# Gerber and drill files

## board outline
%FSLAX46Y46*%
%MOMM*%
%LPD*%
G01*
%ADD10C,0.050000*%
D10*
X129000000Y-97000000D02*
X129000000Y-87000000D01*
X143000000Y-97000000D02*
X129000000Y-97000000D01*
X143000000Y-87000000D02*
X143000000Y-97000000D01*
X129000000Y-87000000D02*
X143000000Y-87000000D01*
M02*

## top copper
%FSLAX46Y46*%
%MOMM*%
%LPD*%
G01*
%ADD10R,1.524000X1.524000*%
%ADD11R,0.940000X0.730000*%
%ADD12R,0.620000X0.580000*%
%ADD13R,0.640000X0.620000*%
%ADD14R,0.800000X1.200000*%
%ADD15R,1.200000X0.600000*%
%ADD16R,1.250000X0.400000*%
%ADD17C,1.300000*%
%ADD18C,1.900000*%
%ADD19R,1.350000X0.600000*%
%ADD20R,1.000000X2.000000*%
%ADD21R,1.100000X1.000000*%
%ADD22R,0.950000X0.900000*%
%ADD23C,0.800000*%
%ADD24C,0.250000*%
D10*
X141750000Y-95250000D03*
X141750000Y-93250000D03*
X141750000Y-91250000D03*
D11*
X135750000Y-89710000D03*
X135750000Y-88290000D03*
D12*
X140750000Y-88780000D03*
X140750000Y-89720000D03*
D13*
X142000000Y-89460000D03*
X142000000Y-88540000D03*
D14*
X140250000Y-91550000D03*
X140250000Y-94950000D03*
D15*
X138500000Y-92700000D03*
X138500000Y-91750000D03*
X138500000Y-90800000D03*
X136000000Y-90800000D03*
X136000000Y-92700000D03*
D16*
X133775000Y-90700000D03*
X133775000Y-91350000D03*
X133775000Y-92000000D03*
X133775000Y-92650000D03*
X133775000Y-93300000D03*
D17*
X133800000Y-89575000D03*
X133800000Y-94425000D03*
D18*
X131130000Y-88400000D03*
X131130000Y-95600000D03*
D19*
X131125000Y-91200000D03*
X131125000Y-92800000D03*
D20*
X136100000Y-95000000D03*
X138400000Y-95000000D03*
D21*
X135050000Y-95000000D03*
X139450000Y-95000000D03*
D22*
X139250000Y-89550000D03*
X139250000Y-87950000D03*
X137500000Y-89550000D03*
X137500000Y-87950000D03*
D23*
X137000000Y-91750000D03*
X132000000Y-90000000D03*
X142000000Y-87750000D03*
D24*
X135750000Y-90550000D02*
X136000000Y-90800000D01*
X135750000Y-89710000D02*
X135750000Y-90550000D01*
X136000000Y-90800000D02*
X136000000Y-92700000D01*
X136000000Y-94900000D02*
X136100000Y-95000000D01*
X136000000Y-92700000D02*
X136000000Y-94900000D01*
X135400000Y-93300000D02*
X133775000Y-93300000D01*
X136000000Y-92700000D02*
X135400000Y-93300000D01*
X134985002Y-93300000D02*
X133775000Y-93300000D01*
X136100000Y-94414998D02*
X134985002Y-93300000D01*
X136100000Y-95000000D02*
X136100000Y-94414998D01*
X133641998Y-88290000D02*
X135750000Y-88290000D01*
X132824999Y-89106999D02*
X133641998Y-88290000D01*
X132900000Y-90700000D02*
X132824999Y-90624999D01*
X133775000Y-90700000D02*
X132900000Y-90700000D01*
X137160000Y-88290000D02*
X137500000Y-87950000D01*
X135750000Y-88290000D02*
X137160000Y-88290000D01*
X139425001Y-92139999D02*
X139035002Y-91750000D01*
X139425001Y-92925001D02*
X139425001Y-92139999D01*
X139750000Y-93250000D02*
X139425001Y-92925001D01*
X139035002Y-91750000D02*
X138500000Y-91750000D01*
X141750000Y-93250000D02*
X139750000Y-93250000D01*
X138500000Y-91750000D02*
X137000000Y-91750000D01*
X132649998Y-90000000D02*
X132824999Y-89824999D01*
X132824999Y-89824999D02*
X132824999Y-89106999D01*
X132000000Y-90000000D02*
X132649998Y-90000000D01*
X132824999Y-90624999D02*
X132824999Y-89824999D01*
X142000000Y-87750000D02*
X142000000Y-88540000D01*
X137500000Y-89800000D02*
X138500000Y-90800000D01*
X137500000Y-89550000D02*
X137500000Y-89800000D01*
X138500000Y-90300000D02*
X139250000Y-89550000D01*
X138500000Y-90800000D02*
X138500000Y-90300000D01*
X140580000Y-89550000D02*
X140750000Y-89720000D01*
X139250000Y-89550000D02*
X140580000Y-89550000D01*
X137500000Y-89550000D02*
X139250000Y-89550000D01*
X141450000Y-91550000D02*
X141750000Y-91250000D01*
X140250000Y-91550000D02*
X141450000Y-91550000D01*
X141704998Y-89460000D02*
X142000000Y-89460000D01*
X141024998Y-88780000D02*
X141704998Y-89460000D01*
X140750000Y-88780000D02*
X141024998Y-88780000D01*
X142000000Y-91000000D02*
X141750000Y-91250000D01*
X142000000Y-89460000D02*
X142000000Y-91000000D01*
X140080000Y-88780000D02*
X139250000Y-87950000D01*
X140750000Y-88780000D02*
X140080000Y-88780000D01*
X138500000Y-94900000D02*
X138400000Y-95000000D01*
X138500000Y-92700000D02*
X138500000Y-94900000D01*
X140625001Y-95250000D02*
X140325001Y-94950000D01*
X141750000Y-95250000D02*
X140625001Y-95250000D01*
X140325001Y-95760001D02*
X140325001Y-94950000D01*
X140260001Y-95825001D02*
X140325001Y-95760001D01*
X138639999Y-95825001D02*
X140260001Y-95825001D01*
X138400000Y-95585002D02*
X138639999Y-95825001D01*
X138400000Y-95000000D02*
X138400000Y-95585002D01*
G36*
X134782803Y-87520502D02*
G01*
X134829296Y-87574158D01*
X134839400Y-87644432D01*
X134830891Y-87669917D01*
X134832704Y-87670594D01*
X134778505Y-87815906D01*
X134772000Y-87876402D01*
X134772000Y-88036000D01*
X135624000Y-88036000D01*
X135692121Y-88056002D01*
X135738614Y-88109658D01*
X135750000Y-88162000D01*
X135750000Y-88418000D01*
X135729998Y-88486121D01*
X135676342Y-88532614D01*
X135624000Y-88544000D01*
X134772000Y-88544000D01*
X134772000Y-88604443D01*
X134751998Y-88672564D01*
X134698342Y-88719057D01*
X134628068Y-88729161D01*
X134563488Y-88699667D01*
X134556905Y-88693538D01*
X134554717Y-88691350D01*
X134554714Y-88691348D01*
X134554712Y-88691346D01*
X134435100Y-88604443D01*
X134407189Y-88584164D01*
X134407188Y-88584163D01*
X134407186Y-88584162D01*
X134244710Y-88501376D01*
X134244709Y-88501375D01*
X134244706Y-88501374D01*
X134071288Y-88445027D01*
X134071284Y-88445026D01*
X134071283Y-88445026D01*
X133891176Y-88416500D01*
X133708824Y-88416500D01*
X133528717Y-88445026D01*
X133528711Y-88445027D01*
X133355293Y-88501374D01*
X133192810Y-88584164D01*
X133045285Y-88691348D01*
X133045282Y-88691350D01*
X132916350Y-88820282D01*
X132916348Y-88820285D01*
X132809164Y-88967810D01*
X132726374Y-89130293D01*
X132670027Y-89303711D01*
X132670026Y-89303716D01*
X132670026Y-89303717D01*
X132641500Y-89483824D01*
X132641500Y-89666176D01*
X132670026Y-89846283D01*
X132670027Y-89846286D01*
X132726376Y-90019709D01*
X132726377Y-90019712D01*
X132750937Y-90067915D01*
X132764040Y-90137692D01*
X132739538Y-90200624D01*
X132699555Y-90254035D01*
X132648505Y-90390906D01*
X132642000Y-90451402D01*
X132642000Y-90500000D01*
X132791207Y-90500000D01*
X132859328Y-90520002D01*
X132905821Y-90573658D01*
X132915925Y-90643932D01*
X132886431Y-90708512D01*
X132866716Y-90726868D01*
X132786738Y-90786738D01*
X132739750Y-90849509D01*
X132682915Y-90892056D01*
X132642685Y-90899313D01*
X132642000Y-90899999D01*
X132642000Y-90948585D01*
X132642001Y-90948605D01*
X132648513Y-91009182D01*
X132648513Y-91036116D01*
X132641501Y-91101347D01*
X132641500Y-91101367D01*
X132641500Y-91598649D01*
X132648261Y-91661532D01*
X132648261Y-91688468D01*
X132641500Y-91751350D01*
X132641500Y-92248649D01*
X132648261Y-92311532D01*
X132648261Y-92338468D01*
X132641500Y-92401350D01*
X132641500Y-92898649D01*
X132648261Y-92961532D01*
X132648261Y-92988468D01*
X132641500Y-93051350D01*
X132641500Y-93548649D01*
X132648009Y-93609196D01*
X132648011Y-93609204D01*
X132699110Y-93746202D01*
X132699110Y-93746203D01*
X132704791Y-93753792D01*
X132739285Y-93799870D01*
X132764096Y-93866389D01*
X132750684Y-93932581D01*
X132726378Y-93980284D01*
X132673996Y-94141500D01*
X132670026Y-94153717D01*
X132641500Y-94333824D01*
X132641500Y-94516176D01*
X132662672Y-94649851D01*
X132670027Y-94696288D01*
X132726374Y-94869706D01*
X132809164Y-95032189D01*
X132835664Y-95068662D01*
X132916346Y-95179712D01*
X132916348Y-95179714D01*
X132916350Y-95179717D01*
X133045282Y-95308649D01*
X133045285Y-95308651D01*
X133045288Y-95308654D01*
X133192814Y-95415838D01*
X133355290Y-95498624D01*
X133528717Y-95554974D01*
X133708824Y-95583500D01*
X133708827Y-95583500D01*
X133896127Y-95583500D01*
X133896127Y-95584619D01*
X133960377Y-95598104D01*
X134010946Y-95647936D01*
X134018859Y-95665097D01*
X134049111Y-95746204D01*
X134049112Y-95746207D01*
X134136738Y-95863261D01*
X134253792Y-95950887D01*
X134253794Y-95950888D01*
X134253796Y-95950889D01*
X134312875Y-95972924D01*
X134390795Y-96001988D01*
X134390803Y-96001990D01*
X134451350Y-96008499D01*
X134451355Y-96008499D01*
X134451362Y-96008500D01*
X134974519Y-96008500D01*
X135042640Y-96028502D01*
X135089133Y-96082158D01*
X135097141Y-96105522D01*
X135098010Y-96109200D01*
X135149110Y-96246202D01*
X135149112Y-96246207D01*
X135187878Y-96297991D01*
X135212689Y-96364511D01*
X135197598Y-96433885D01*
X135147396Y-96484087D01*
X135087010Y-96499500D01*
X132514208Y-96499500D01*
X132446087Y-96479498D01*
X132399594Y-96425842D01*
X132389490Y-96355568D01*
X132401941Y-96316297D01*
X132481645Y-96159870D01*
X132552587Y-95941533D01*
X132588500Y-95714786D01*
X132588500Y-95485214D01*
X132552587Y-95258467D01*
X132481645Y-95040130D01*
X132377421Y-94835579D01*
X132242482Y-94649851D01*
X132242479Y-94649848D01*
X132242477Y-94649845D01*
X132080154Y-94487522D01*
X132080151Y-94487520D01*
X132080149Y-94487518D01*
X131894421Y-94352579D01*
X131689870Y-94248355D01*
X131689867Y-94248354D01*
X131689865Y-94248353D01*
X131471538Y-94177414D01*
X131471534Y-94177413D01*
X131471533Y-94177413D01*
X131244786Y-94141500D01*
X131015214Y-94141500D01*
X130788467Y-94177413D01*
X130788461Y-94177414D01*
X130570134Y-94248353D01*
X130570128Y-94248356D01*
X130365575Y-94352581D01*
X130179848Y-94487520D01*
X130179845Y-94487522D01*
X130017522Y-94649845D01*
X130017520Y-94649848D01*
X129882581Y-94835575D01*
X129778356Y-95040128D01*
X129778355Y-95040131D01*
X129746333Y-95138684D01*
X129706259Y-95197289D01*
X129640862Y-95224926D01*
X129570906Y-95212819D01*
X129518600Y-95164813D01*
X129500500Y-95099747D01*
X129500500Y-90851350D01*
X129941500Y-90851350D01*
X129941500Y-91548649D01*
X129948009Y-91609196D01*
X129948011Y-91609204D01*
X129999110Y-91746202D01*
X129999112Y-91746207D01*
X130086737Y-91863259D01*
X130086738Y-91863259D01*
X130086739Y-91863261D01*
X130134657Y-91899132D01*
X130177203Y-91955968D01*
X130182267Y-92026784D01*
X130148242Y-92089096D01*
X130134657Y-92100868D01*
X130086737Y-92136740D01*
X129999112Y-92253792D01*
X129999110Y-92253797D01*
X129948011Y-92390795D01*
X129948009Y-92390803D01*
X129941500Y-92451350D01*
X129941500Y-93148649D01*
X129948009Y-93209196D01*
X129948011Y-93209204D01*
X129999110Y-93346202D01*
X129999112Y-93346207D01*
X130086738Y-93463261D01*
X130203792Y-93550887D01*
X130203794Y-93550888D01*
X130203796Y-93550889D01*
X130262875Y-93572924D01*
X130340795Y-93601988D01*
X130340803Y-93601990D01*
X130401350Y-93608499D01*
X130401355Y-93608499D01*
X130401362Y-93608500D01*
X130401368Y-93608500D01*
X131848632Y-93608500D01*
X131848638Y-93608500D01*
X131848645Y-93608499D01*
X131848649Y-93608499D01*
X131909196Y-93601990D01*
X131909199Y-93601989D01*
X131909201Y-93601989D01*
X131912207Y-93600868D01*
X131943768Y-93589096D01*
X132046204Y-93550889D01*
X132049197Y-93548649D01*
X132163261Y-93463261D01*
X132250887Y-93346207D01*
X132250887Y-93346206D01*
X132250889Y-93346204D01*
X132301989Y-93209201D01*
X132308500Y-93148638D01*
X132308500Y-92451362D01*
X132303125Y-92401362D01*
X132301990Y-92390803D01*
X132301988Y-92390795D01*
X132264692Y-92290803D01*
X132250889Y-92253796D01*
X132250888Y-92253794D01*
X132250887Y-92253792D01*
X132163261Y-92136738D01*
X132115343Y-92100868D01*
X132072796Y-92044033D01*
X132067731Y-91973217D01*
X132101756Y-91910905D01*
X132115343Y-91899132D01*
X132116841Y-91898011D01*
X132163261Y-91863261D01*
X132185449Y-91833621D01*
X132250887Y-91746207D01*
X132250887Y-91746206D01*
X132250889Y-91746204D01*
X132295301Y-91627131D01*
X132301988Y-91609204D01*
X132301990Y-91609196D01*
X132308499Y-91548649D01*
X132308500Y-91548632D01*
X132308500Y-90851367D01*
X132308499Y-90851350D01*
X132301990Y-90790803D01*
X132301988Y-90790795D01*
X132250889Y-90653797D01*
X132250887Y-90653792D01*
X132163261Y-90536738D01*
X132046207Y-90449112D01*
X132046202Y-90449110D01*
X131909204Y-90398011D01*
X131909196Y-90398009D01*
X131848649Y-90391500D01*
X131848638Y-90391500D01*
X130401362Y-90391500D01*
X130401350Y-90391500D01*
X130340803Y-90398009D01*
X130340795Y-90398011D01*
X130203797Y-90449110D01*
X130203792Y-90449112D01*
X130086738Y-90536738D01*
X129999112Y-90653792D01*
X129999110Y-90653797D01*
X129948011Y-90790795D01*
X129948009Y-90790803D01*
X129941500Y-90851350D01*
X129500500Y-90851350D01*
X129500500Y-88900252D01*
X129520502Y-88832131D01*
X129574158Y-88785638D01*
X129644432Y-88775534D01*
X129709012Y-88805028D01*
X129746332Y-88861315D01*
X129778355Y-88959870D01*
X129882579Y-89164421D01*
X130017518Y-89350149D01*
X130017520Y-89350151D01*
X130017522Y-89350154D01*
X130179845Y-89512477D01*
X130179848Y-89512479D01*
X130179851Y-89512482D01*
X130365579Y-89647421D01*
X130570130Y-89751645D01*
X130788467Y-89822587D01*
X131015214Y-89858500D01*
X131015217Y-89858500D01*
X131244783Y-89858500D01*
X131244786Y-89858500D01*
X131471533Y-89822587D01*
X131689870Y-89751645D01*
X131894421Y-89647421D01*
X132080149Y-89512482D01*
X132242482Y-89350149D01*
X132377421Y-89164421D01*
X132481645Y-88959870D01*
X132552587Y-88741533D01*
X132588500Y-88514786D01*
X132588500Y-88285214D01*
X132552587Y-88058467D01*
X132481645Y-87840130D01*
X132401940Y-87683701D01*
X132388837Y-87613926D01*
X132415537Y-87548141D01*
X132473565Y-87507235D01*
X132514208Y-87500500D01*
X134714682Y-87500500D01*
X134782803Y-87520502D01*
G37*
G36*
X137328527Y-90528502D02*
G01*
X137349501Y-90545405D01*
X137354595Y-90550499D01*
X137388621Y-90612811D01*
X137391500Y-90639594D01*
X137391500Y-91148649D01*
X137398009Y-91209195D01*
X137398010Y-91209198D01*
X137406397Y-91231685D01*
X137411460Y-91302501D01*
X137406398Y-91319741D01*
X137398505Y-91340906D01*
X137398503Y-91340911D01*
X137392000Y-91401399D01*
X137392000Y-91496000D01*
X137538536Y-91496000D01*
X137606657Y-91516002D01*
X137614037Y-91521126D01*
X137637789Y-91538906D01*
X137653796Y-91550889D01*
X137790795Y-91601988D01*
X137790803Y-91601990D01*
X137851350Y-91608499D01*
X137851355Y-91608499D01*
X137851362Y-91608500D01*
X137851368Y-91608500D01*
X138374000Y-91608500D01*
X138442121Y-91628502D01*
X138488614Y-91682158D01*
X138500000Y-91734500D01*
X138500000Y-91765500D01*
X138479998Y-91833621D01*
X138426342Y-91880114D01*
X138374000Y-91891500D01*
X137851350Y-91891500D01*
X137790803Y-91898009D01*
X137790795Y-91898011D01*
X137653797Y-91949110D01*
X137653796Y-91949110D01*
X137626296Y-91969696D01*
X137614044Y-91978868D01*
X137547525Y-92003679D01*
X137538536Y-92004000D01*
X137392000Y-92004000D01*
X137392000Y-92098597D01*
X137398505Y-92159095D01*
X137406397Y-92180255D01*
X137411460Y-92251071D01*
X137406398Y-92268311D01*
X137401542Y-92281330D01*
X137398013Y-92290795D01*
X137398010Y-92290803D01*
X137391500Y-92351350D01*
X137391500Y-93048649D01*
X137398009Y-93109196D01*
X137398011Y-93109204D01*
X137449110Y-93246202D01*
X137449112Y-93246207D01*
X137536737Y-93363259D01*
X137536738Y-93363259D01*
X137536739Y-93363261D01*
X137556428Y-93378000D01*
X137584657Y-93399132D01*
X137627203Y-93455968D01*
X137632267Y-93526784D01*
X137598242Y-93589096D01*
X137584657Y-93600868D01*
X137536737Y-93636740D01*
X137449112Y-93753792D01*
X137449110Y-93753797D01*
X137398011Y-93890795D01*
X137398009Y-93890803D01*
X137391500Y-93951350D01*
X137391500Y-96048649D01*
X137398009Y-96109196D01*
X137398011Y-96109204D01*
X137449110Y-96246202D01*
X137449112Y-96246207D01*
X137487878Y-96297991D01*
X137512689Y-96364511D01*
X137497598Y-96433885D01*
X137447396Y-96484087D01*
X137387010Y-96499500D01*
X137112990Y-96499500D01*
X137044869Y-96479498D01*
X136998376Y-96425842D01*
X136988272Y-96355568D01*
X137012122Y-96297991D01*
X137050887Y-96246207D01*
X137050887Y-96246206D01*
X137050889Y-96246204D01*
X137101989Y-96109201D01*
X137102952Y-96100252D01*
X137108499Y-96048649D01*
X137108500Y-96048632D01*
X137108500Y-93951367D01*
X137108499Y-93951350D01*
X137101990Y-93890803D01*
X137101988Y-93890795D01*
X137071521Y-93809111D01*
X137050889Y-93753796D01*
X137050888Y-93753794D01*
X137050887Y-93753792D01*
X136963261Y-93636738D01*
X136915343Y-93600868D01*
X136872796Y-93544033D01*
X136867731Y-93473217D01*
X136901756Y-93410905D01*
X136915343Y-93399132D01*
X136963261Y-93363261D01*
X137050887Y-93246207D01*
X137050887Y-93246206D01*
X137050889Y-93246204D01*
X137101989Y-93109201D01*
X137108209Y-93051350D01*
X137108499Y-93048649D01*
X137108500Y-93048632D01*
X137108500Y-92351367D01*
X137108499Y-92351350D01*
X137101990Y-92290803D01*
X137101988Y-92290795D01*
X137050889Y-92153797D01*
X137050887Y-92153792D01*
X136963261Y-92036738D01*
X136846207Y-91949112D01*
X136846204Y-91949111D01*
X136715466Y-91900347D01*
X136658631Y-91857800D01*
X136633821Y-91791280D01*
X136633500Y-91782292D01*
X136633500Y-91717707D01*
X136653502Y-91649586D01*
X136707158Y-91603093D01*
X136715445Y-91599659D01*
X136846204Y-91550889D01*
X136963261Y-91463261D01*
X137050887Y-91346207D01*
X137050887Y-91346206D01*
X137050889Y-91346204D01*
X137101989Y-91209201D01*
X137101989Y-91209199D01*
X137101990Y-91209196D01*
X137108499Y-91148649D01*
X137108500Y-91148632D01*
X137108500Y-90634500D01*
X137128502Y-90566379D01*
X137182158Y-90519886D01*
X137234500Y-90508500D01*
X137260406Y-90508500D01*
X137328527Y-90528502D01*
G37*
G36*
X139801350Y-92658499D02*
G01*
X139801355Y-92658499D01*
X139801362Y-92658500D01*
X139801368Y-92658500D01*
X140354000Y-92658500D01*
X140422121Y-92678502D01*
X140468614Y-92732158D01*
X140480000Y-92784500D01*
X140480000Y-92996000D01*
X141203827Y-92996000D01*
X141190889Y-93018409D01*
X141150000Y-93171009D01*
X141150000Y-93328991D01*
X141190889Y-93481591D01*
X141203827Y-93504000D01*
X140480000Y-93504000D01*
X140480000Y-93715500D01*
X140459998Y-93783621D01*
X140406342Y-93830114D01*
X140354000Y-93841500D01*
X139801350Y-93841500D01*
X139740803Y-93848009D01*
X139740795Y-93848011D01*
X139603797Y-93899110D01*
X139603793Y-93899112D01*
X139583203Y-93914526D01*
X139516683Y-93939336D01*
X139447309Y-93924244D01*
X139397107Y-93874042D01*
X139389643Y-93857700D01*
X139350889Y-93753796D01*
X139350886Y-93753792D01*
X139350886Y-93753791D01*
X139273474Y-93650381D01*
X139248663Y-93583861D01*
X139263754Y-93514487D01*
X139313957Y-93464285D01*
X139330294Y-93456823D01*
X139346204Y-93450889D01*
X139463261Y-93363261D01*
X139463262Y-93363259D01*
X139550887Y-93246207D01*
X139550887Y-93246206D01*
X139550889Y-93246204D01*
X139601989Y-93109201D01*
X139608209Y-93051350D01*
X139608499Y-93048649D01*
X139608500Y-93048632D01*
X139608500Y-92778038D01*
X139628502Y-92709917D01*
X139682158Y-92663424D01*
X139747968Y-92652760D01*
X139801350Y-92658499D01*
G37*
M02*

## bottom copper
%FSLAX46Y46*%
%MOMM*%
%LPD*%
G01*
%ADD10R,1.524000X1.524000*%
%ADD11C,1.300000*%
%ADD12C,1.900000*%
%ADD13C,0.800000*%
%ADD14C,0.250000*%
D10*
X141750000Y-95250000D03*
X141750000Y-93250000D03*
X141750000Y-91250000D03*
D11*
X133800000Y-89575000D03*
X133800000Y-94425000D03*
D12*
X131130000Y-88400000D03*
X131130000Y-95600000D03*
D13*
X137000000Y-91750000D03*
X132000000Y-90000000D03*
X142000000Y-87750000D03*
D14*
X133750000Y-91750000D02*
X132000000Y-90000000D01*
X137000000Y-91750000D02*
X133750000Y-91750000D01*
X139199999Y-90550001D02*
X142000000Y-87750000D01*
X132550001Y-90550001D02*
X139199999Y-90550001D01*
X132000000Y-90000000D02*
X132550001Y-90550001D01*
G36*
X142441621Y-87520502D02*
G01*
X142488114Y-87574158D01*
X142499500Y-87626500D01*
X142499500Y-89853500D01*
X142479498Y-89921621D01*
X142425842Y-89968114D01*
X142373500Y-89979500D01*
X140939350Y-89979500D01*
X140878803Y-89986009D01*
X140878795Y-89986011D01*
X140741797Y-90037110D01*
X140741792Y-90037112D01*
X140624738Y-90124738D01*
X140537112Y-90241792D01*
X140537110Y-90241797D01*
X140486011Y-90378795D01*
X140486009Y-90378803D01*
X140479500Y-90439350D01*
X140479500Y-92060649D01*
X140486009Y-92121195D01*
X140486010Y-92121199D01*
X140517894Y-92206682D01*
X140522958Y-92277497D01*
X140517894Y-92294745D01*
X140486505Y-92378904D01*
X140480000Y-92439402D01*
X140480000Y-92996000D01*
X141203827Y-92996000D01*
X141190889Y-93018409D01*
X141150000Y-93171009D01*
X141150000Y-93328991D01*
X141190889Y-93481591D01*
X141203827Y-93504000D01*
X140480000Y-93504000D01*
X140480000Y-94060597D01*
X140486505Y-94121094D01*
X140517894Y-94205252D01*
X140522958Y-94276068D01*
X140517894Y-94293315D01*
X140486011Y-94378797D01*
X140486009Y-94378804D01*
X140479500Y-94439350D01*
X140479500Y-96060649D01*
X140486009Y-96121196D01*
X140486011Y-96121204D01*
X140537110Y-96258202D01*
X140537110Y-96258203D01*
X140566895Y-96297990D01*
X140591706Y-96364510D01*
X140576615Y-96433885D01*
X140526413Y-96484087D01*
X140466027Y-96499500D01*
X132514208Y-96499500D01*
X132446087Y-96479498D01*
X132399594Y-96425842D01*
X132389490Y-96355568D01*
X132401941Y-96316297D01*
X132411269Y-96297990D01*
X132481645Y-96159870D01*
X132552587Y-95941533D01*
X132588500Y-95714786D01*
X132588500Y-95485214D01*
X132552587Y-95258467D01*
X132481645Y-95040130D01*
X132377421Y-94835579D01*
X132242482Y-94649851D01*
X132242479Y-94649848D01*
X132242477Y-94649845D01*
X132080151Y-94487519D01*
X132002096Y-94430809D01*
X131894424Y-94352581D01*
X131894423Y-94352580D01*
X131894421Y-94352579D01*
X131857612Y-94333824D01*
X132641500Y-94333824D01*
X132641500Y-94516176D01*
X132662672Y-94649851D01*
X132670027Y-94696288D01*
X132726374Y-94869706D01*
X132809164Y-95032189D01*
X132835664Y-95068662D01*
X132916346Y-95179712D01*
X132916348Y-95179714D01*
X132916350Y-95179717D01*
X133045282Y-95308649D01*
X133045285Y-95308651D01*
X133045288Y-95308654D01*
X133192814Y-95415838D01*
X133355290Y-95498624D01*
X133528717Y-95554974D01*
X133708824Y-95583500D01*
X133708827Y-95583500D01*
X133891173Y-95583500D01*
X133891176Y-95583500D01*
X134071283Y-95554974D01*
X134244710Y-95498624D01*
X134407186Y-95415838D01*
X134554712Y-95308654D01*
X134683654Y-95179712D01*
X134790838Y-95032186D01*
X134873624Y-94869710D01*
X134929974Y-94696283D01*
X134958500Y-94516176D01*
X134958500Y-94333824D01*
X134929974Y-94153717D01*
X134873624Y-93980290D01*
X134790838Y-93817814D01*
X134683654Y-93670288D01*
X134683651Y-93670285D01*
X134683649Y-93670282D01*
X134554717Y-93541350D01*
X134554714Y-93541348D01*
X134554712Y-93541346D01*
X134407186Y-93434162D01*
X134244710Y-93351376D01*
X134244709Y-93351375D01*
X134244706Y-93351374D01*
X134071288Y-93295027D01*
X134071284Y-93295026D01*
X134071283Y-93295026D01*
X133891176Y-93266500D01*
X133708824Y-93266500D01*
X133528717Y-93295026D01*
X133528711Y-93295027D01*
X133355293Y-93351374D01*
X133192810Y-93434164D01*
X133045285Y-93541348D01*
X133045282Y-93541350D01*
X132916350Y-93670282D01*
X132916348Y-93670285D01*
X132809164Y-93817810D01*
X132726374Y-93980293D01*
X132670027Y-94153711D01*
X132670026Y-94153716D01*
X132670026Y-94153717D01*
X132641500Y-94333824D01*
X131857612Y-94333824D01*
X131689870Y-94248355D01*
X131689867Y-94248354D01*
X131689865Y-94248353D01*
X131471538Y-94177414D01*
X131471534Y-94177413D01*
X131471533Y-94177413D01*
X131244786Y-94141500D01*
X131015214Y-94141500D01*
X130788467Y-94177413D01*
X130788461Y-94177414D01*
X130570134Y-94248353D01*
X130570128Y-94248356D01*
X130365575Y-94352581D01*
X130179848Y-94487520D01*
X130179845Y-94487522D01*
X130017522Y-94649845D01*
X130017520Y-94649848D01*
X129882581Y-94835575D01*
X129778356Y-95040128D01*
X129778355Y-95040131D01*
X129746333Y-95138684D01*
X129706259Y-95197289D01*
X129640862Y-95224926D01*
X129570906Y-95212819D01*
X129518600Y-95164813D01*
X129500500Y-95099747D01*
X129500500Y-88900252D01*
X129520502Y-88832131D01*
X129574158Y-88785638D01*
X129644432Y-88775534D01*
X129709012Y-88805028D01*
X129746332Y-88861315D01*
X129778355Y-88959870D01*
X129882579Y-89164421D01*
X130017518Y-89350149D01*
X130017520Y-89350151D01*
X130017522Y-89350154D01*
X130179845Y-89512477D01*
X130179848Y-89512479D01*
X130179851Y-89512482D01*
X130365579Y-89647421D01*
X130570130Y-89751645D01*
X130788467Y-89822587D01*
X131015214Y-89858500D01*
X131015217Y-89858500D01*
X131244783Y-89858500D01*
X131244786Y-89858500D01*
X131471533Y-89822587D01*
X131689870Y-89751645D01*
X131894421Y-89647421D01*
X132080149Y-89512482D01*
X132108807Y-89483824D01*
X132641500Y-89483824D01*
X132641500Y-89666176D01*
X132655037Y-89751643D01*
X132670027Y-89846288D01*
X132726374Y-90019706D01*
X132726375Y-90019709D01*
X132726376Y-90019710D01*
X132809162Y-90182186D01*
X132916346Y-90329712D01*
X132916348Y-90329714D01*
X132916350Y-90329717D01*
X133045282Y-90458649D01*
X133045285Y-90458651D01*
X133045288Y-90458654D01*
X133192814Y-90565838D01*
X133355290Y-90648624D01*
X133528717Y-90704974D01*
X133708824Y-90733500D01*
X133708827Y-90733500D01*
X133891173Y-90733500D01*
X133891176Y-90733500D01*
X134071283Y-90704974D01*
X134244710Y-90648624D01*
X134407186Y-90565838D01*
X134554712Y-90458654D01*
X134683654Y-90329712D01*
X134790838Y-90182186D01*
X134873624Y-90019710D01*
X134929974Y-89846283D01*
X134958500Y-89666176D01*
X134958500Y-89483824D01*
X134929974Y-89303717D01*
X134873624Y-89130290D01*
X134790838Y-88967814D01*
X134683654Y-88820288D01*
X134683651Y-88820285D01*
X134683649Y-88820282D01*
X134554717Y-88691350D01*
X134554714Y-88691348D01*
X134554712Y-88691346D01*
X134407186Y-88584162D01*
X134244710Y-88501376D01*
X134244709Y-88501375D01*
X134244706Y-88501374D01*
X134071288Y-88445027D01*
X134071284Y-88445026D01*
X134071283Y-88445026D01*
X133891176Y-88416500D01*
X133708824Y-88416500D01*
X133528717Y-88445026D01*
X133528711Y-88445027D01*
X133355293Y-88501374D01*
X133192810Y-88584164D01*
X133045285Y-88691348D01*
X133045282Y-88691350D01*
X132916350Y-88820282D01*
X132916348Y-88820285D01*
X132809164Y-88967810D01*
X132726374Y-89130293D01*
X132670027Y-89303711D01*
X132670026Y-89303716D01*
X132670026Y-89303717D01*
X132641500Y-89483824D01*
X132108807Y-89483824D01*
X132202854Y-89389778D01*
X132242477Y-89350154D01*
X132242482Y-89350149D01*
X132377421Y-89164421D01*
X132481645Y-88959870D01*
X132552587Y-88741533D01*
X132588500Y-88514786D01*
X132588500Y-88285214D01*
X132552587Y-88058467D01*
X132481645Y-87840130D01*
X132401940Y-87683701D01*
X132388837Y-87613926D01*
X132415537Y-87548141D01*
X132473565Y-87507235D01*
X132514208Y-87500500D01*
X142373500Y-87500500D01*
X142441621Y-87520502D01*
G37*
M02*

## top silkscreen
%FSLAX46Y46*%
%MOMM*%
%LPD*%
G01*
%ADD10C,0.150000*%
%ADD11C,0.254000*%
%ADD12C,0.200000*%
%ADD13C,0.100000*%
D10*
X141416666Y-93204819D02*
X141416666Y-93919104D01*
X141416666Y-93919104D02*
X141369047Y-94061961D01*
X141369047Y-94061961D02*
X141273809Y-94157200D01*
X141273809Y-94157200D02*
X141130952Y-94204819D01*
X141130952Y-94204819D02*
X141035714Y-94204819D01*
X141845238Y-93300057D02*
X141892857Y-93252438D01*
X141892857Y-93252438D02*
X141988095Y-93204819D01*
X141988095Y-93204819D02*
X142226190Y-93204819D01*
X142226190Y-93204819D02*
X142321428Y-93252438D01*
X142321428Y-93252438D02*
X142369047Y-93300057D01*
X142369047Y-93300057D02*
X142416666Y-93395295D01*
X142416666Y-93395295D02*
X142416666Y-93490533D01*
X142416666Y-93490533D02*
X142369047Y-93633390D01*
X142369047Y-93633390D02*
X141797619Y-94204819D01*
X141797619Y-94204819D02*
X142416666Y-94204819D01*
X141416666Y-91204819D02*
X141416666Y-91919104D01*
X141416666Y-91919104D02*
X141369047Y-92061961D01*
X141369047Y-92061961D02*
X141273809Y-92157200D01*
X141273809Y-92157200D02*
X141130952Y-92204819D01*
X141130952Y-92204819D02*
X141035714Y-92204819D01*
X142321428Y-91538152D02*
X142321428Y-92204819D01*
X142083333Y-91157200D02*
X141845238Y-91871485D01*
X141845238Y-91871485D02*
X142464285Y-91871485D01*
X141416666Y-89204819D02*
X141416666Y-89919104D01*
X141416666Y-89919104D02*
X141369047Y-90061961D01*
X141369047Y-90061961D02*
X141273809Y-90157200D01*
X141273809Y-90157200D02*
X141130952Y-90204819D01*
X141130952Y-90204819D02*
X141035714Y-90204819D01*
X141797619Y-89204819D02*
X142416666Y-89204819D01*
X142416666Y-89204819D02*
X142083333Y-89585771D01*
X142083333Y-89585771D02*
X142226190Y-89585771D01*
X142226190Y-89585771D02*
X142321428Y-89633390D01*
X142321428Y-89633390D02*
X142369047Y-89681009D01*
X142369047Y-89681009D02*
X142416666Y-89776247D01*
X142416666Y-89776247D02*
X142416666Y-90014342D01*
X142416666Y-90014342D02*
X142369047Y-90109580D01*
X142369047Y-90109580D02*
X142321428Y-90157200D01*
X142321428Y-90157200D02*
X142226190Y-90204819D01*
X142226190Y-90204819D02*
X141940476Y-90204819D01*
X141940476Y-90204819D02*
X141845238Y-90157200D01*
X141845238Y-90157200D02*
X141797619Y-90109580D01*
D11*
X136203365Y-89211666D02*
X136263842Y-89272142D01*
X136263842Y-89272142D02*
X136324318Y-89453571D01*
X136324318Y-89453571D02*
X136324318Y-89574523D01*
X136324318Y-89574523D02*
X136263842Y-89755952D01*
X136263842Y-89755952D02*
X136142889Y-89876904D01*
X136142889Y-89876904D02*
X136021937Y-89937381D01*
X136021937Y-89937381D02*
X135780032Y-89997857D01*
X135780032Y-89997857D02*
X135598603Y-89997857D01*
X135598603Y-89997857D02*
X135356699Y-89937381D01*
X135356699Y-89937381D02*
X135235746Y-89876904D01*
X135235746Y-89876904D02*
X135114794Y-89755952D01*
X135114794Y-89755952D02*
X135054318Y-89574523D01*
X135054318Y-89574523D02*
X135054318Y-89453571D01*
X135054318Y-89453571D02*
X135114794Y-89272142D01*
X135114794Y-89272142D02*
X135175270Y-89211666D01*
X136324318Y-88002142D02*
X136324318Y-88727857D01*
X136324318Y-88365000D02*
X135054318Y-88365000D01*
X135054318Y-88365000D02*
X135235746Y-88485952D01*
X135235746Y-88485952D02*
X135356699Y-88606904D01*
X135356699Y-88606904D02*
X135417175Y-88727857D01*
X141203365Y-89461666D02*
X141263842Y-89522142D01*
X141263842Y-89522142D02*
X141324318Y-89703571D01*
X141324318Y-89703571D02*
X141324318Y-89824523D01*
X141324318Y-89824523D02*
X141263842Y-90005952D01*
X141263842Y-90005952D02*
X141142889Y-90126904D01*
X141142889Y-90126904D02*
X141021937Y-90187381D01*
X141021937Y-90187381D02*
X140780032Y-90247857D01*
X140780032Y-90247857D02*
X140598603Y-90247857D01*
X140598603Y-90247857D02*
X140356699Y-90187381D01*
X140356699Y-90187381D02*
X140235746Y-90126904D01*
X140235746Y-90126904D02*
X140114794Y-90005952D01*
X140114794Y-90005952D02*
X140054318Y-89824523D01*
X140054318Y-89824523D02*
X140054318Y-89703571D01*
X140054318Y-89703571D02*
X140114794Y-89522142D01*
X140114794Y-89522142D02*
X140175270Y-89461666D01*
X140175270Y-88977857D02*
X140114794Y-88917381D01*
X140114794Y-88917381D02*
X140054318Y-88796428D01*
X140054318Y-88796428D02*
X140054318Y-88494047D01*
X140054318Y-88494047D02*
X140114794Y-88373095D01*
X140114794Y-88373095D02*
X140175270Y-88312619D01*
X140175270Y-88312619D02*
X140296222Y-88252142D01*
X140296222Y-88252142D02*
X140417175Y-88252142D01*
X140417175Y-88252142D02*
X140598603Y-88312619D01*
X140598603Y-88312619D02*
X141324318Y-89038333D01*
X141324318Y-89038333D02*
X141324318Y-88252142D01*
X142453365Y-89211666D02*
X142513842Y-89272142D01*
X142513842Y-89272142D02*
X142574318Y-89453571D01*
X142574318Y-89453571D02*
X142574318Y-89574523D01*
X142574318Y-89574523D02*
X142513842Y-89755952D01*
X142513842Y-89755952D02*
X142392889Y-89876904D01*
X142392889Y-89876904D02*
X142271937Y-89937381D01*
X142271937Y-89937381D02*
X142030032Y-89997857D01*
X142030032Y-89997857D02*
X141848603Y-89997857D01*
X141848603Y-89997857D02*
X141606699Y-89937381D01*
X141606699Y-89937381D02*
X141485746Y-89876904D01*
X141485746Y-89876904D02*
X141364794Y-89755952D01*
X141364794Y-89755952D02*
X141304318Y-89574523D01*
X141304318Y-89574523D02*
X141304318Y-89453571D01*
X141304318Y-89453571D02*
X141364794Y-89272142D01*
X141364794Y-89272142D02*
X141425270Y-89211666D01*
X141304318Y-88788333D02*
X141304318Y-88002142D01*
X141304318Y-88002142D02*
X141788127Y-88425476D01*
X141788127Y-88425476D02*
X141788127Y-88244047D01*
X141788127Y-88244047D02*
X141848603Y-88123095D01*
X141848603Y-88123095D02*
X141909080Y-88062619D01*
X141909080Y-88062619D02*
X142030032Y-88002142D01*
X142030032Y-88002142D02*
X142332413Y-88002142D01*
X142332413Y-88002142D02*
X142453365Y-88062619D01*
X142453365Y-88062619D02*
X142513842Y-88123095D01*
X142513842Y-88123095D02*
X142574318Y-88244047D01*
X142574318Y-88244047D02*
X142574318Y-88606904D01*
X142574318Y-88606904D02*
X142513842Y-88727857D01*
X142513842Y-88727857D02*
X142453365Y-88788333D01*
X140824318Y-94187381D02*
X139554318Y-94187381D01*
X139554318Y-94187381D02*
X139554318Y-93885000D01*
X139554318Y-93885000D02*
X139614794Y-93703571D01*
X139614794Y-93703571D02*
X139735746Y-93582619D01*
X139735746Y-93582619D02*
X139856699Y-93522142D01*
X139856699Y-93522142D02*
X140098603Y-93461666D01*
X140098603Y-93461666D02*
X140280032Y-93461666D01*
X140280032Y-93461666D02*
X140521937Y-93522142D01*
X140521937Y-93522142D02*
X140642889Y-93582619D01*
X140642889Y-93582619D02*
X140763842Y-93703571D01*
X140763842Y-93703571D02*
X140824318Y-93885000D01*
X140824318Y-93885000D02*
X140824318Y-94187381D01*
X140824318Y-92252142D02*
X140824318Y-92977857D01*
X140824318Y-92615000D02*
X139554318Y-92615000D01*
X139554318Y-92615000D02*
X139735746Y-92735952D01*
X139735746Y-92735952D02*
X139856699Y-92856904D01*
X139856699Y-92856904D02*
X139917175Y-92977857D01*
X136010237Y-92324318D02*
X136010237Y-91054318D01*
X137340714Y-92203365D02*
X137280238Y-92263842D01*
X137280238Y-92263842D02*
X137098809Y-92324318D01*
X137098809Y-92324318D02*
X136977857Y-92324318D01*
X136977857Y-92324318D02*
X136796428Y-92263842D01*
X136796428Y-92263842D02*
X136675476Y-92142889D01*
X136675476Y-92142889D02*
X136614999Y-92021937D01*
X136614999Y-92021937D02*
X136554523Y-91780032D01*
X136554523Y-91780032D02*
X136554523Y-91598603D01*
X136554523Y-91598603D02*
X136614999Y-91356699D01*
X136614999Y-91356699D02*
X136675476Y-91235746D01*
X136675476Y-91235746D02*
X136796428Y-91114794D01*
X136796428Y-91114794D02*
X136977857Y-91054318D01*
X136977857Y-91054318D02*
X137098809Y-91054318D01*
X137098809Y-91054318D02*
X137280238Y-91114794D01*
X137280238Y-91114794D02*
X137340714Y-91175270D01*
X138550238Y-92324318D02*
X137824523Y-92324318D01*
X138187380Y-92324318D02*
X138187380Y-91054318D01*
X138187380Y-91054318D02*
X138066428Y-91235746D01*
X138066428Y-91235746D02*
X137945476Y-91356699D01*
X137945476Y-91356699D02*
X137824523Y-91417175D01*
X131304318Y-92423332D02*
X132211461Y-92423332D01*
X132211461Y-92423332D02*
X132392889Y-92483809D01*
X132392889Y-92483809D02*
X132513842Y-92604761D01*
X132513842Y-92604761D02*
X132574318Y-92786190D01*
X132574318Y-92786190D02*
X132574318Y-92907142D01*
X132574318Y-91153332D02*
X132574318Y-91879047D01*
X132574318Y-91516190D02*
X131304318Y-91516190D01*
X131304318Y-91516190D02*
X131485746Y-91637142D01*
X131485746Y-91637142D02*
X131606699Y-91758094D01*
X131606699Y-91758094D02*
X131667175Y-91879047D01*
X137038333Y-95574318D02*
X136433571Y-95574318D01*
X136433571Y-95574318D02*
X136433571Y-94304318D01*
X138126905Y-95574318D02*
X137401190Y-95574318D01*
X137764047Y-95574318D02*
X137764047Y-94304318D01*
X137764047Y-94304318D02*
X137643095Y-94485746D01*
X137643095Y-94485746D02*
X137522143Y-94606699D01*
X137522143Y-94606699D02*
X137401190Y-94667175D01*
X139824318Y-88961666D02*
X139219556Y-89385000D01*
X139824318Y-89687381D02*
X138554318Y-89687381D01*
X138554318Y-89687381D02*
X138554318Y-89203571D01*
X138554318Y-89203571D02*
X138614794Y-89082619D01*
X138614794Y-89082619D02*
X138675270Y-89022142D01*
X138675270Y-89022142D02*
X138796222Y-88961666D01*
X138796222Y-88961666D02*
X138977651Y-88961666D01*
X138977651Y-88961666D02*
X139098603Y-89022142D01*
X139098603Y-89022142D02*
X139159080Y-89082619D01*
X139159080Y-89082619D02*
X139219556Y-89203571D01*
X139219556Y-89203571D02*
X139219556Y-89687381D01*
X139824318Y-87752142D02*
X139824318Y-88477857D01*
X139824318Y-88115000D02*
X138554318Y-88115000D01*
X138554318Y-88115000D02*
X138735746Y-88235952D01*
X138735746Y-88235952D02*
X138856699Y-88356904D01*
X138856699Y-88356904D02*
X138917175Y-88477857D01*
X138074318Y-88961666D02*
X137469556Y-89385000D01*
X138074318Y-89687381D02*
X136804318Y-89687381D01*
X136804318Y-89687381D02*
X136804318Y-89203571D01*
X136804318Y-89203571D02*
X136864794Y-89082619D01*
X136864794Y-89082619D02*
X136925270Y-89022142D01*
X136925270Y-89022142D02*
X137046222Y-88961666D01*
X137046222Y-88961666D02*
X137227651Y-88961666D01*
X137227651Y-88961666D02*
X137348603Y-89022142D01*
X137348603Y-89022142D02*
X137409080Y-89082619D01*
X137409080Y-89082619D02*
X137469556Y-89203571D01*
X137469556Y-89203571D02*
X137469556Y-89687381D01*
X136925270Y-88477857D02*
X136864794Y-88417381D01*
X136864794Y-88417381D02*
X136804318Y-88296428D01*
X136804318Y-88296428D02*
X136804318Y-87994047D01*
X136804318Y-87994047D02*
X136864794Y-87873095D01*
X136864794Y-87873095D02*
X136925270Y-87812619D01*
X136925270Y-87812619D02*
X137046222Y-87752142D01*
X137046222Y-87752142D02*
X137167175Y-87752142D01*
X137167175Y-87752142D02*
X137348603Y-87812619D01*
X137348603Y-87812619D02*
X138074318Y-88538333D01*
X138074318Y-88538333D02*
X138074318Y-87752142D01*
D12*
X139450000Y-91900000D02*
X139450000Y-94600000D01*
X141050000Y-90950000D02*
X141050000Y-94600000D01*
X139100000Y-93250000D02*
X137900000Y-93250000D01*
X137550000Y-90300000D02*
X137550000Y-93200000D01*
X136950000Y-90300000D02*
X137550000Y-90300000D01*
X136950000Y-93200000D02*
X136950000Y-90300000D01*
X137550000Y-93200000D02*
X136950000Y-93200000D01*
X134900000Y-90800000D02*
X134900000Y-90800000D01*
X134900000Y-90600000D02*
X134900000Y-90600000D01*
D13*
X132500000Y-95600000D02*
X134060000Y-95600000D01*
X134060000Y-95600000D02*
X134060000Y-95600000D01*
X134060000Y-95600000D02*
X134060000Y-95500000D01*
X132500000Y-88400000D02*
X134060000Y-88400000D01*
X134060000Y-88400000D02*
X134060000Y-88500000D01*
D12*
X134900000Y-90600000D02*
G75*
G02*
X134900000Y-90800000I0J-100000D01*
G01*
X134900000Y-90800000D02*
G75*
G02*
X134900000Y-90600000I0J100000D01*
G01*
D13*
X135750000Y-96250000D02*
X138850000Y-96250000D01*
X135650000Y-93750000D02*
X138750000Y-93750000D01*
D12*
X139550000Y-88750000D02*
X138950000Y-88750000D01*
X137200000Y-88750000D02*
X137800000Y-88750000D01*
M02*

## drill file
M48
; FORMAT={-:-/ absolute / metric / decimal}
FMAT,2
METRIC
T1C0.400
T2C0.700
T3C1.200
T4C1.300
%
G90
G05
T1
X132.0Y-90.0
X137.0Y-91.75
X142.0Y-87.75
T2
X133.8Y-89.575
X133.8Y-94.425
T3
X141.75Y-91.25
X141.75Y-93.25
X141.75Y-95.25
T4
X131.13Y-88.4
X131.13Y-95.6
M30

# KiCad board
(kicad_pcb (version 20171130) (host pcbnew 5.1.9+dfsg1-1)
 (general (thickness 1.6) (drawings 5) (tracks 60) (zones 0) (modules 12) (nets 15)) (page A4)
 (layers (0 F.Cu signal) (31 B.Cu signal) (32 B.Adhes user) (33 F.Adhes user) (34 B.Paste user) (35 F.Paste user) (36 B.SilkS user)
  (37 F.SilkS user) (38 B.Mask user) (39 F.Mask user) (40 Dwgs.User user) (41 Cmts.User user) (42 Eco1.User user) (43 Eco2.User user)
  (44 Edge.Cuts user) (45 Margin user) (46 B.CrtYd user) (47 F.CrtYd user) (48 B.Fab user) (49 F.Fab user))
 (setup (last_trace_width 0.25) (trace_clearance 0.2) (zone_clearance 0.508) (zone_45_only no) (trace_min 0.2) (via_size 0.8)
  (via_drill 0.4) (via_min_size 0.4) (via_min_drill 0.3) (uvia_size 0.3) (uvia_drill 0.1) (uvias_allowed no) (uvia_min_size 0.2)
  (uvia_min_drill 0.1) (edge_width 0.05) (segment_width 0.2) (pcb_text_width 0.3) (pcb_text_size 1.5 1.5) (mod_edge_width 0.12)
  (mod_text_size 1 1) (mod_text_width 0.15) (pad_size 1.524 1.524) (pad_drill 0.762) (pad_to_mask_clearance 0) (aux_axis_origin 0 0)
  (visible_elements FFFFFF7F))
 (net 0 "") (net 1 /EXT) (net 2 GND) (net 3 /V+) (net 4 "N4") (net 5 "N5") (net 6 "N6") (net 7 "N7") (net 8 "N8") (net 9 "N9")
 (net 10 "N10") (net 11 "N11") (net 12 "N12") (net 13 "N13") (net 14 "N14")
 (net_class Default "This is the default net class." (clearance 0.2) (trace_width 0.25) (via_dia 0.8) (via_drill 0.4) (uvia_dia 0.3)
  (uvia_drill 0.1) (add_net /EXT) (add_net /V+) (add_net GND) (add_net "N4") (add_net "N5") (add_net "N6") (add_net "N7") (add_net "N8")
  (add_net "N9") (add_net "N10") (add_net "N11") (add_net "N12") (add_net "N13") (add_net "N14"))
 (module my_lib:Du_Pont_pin (layer F.Cu) (at 141.75 95.25)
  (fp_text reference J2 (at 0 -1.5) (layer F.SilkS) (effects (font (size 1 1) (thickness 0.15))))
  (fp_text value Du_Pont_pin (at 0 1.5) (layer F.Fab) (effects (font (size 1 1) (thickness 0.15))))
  (pad 1 thru_hole rect (at 0 0) (size 1.524 1.524) (drill 1.2) (layers *.Cu *.Mask) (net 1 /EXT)))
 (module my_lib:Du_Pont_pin (layer F.Cu) (at 141.75 93.25)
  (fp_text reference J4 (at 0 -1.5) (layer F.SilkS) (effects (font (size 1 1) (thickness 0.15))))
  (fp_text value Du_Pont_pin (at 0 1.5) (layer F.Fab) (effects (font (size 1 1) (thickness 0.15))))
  (pad 1 thru_hole rect (at 0 0) (size 1.524 1.524) (drill 1.2) (layers *.Cu *.Mask) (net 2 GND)))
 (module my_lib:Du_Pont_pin (layer F.Cu) (at 141.75 91.25)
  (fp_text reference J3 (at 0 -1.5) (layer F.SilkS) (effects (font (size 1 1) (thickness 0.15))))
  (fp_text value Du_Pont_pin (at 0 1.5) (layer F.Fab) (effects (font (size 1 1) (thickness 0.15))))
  (pad 1 thru_hole rect (at 0 0) (size 1.524 1.524) (drill 1.2) (layers *.Cu *.Mask) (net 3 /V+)))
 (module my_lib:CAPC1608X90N (layer F.Cu) (at 135.75 89 90)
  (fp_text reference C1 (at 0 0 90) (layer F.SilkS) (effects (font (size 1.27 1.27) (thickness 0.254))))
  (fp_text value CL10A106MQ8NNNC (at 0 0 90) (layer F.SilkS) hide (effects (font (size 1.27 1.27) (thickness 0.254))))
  (pad 1 smd rect (at -0.71 0 90) (size 0.73 0.94) (layers F.Cu F.Paste F.Mask) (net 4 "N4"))
  (pad 2 smd rect (at 0.71 0 90) (size 0.73 0.94) (layers F.Cu F.Paste F.Mask) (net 2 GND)))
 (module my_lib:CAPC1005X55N (layer F.Cu) (at 140.75 89.25 270)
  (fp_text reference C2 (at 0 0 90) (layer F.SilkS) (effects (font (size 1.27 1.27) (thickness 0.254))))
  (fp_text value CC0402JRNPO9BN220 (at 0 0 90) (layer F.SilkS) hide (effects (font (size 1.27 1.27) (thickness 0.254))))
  (pad 1 smd rect (at -0.47 0 270) (size 0.58 0.62) (layers F.Cu F.Paste F.Mask) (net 3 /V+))
  (pad 2 smd rect (at 0.47 0 270) (size 0.58 0.62) (layers F.Cu F.Paste F.Mask) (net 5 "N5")))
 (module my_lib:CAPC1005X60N (layer F.Cu) (at 142 89 90)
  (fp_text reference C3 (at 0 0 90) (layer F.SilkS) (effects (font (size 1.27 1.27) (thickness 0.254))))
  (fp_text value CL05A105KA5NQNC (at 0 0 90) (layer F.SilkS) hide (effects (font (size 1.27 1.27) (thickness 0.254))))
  (pad 1 smd rect (at -0.46 0 90) (size 0.62 0.64) (layers F.Cu F.Paste F.Mask) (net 3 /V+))
  (pad 2 smd rect (at 0.46 0 90) (size 0.62 0.64) (layers F.Cu F.Paste F.Mask) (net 2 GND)))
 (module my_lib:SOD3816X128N (layer F.Cu) (at 140.25 93.25 270)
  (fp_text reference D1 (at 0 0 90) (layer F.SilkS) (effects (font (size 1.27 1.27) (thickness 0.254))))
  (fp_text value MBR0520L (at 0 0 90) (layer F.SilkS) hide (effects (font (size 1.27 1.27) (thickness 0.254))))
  (fp_line (start -1.35 0.8) (end 1.35 0.8) (layer F.SilkS) (width 0.2))
  (fp_line (start -2.3 -0.8) (end 1.35 -0.8) (layer F.SilkS) (width 0.2))
  (pad 1 smd rect (at -1.7 0) (size 0.8 1.2) (layers F.Cu F.Paste F.Mask) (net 3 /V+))
  (pad 2 smd rect (at 1.7 0) (size 0.8 1.2) (layers F.Cu F.Paste F.Mask) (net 1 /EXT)))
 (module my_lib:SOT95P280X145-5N (layer F.Cu) (at 137.25 91.75 180)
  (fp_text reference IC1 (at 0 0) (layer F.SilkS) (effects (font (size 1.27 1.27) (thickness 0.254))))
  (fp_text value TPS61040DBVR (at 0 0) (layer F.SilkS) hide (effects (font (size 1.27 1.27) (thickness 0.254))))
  (fp_line (start -1.85 -1.5) (end -0.65 -1.5) (layer F.SilkS) (width 0.2))
  (fp_line (start -0.3 1.45) (end -0.3 -1.45) (layer F.SilkS) (width 0.2))
  (fp_line (start 0.3 1.45) (end -0.3 1.45) (layer F.SilkS) (width 0.2))
  (fp_line (start 0.3 -1.45) (end 0.3 1.45) (layer F.SilkS) (width 0.2))
  (fp_line (start -0.3 -1.45) (end 0.3 -1.45) (layer F.SilkS) (width 0.2))
  (pad 1 smd rect (at -1.25 -0.95 270) (size 0.6 1.2) (layers F.Cu F.Paste F.Mask) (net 1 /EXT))
  (pad 2 smd rect (at -1.25 0 270) (size 0.6 1.2) (layers F.Cu F.Paste F.Mask) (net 2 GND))
  (pad 3 smd rect (at -1.25 0.95 270) (size 0.6 1.2) (layers F.Cu F.Paste F.Mask) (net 5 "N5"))
  (pad 4 smd rect (at 1.25 0.95 270) (size 0.6 1.2) (layers F.Cu F.Paste F.Mask) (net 4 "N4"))
  (pad 5 smd rect (at 1.25 -0.95 270) (size 0.6 1.2) (layers F.Cu F.Paste F.Mask) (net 4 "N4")))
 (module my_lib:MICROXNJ (layer F.Cu) (at 129 92 90)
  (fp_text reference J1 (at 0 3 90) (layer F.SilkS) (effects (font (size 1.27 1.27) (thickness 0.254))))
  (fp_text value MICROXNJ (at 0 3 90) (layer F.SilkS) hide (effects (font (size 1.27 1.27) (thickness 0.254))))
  (fp_line (start 1.2 5.9) (end 1.2 5.9) (layer F.SilkS) (width 0.2))
  (fp_line (start 1.4 5.9) (end 1.4 5.9) (layer F.SilkS) (width 0.2))
  (fp_line (start -3.6 3.5) (end -3.6 5.06) (layer F.SilkS) (width 0.1))
  (fp_line (start -3.6 5.06) (end -3.6 5.06) (layer F.SilkS) (width 0.1))
  (fp_line (start -3.6 5.06) (end -3.5 5.06) (layer F.SilkS) (width 0.1))
  (fp_line (start 3.6 3.5) (end 3.6 5.06) (layer F.SilkS) (width 0.1))
  (fp_line (start 3.6 5.06) (end 3.5 5.06) (layer F.SilkS) (width 0.1))
  (fp_arc (start 1.3 5.9) (end 1.2 5.9) (angle -180) (layer F.SilkS) (width 0.2))
  (fp_arc (start 1.3 5.9) (end 1.4 5.9) (angle -180) (layer F.SilkS) (width 0.2))
  (pad 1 smd rect (at 1.3 4.775 90) (size 0.4 1.25) (layers F.Cu F.Paste F.Mask) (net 2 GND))
  (pad 2 smd rect (at 0.65 4.775 90) (size 0.4 1.25) (layers F.Cu F.Paste F.Mask) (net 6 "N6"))
  (pad 3 smd rect (at 0 4.775 90) (size 0.4 1.25) (layers F.Cu F.Paste F.Mask) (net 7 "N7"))
  (pad 4 smd rect (at -0.65 4.775 90) (size 0.4 1.25) (layers F.Cu F.Paste F.Mask) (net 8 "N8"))
  (pad 5 smd rect (at -1.3 4.775 90) (size 0.4 1.25) (layers F.Cu F.Paste F.Mask) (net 4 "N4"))
  (pad MH1 thru_hole circle (at 2.425 4.8 90) (size 1.3 1.3) (drill 0.7) (layers *.Cu *.Mask) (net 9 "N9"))
  (pad MH2 thru_hole circle (at -2.425 4.8 90) (size 1.3 1.3) (drill 0.7) (layers *.Cu *.Mask) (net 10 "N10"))
  (pad MH3 thru_hole circle (at 3.6 2.13 90) (size 1.9 1.9) (drill 1.3) (layers *.Cu *.Mask) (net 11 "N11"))
  (pad MH4 thru_hole circle (at -3.6 2.13 90) (size 1.9 1.9) (drill 1.3) (layers *.Cu *.Mask) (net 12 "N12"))
  (pad MP1 smd rect (at 0.8 2.125 90) (size 0.6 1.35) (layers F.Cu F.Paste F.Mask) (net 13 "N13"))
  (pad MP2 smd rect (at -0.8 2.125 90) (size 0.6 1.35) (layers F.Cu F.Paste F.Mask) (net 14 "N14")))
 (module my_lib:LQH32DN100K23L (layer F.Cu) (at 137.25 95)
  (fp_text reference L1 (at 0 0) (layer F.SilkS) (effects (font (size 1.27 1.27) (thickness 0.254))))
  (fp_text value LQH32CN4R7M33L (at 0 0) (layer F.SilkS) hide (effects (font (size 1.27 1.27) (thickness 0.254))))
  (fp_line (start -1.5 1.25) (end 1.6 1.25) (layer F.SilkS) (width 0.1))
  (fp_line (start -1.6 -1.25) (end 1.5 -1.25) (layer F.SilkS) (width 0.1))
  (pad 1 smd rect (at -1.15 0) (size 1 2) (layers F.Cu F.Paste F.Mask) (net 4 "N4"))
  (pad 2 smd rect (at 1.15 0) (size 1 2) (layers F.Cu F.Paste F.Mask) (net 1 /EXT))
  (pad 3 smd rect (at -2.2 0 90) (size 1 1.1) (layers F.Cu F.Paste F.Mask))
  (pad 4 smd rect (at 2.2 0 90) (size 1 1.1) (layers F.Cu F.Paste F.Mask)))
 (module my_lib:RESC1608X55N (layer F.Cu) (at 139.25 88.75 270)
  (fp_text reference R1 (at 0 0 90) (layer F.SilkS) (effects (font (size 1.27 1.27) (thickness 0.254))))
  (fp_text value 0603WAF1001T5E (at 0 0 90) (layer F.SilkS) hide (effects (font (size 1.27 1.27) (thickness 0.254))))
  (fp_line (start 0 -0.3) (end 0 0.3) (layer F.SilkS) (width 0.2))
  (pad 2 smd rect (at 0.8 0 270) (size 0.9 0.95) (layers F.Cu F.Paste F.Mask) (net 5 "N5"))
  (pad 1 smd rect (at -0.8 0 270) (size 0.9 0.95) (layers F.Cu F.Paste F.Mask) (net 3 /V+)))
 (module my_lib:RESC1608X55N (layer F.Cu) (at 137.5 88.75 90)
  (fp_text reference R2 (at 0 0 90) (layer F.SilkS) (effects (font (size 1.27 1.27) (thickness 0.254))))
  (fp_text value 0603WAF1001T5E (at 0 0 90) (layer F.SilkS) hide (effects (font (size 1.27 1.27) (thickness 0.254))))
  (fp_line (start 0 -0.3) (end 0 0.3) (layer F.SilkS) (width 0.2))
  (pad 1 smd rect (at -0.8 0 90) (size 0.9 0.95) (layers F.Cu F.Paste F.Mask) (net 5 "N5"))
  (pad 2 smd rect (at 0.8 0 90) (size 0.9 0.95) (layers F.Cu F.Paste F.Mask) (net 2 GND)))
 (gr_line (start 129 97) (end 129 87) (layer Edge.Cuts) (width 0.05))
 (gr_line (start 143 97) (end 129 97) (layer Edge.Cuts) (width 0.05))
 (gr_line (start 143 87) (end 143 97) (layer Edge.Cuts) (width 0.05))
 (gr_line (start 129 87) (end 143 87) (layer Edge.Cuts) (width 0.05))
 (segment (start 135.75 90.55) (end 136 90.8) (width 0.25) (layer F.Cu) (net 4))
 (segment (start 135.75 89.71) (end 135.75 90.55) (width 0.25) (layer F.Cu) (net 4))
 (segment (start 136 90.8) (end 136 92.7) (width 0.25) (layer F.Cu) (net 4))
 (segment (start 136 94.9) (end 136.1 95) (width 0.25) (layer F.Cu) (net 4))
 (segment (start 136 92.7) (end 136 94.9) (width 0.25) (layer F.Cu) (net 4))
 (segment (start 135.4 93.3) (end 133.775 93.3) (width 0.25) (layer F.Cu) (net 4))
 (segment (start 136 92.7) (end 135.4 93.3) (width 0.25) (layer F.Cu) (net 4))
 (segment (start 134.985002 93.3) (end 133.775 93.3) (width 0.25) (layer F.Cu) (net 4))
 (segment (start 136.1 94.414998) (end 134.985002 93.3) (width 0.25) (layer F.Cu) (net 4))
 (segment (start 136.1 95) (end 136.1 94.414998) (width 0.25) (layer F.Cu) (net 4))
 (segment (start 133.641998 88.29) (end 135.75 88.29) (width 0.25) (layer F.Cu) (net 2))
 (segment (start 132.824999 89.106999) (end 133.641998 88.29) (width 0.25) (layer F.Cu) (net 2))
 (segment (start 132.9 90.7) (end 132.824999 90.624999) (width 0.25) (layer F.Cu) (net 2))
 (segment (start 133.775 90.7) (end 132.9 90.7) (width 0.25) (layer F.Cu) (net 2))
 (segment (start 137.16 88.29) (end 137.5 87.95) (width 0.25) (layer F.Cu) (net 2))
 (segment (start 135.75 88.29) (end 137.16 88.29) (width 0.25) (layer F.Cu) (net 2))
 (segment (start 139.425001 92.139999) (end 139.035002 91.75) (width 0.25) (layer F.Cu) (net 2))
 (segment (start 139.425001 92.925001) (end 139.425001 92.139999) (width 0.25) (layer F.Cu) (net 2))
 (segment (start 139.75 93.25) (end 139.425001 92.925001) (width 0.25) (layer F.Cu) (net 2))
 (segment (start 139.035002 91.75) (end 138.5 91.75) (width 0.25) (layer F.Cu) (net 2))
 (segment (start 141.75 93.25) (end 139.75 93.25) (width 0.25) (layer F.Cu) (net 2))
 (via (at 137 91.75) (size 0.8) (drill 0.4) (layers F.Cu B.Cu) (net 2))
 (segment (start 138.5 91.75) (end 137 91.75) (width 0.25) (layer F.Cu) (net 2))
 (via (at 132 90) (size 0.8) (drill 0.4) (layers F.Cu B.Cu) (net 2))
 (segment (start 133.75 91.75) (end 132 90) (width 0.25) (layer B.Cu) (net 2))
 (segment (start 137 91.75) (end 133.75 91.75) (width 0.25) (layer B.Cu) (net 2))
 (segment (start 132.649998 90) (end 132.824999 89.824999) (width 0.25) (layer F.Cu) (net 2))
 (segment (start 132.824999 89.824999) (end 132.824999 89.106999) (width 0.25) (layer F.Cu) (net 2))
 (segment (start 132 90) (end 132.649998 90) (width 0.25) (layer F.Cu) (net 2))
 (segment (start 132.824999 90.624999) (end 132.824999 89.824999) (width 0.25) (layer F.Cu) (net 2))
 (via (at 142 87.75) (size 0.8) (drill 0.4) (layers F.Cu B.Cu) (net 2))
 (segment (start 139.199999 90.550001) (end 142 87.75) (width 0.25) (layer B.Cu) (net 2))
 (segment (start 132.550001 90.550001) (end 139.199999 90.550001) (width 0.25) (layer B.Cu) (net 2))
 (segment (start 132 90) (end 132.550001 90.550001) (width 0.25) (layer B.Cu) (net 2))
 (segment (start 142 87.75) (end 142 88.54) (width 0.25) (layer F.Cu) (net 2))
 (segment (start 137.5 89.8) (end 138.5 90.8) (width 0.25) (layer F.Cu) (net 5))
 (segment (start 137.5 89.55) (end 137.5 89.8) (width 0.25) (layer F.Cu) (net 5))
 (segment (start 138.5 90.3) (end 139.25 89.55) (width 0.25) (layer F.Cu) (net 5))
 (segment (start 138.5 90.8) (end 138.5 90.3) (width 0.25) (layer F.Cu) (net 5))
 (segment (start 140.58 89.55) (end 140.75 89.72) (width 0.25) (layer F.Cu) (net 5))
 (segment (start 139.25 89.55) (end 140.58 89.55) (width 0.25) (layer F.Cu) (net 5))
 (segment (start 137.5 89.55) (end 139.25 89.55) (width 0.25) (layer F.Cu) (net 5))
 (segment (start 141.45 91.55) (end 141.75 91.25) (width 0.25) (layer F.Cu) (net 3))
 (segment (start 140.25 91.55) (end 141.45 91.55) (width 0.25) (layer F.Cu) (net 3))
 (segment (start 141.704998 89.46) (end 142 89.46) (width 0.25) (layer F.Cu) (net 3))
 (segment (start 141.024998 88.78) (end 141.704998 89.46) (width 0.25) (layer F.Cu) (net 3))
 (segment (start 140.75 88.78) (end 141.024998 88.78) (width 0.25) (layer F.Cu) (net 3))
 (segment (start 142 91) (end 141.75 91.25) (width 0.25) (layer F.Cu) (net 3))
 (segment (start 142 89.46) (end 142 91) (width 0.25) (layer F.Cu) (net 3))
 (segment (start 140.08 88.78) (end 139.25 87.95) (width 0.25) (layer F.Cu) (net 3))
 (segment (start 140.75 88.78) (end 140.08 88.78) (width 0.25) (layer F.Cu) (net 3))
 (segment (start 138.5 94.9) (end 138.4 95) (width 0.25) (layer F.Cu) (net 1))
 (segment (start 138.5 92.7) (end 138.5 94.9) (width 0.25) (layer F.Cu) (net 1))
 (segment (start 140.625001 95.25) (end 140.325001 94.95) (width 0.25) (layer F.Cu) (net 1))
 (segment (start 141.75 95.25) (end 140.625001 95.25) (width 0.25) (layer F.Cu) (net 1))
 (segment (start 140.325001 95.760001) (end 140.325001 94.95) (width 0.25) (layer F.Cu) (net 1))
 (segment (start 140.260001 95.825001) (end 140.325001 95.760001) (width 0.25) (layer F.Cu) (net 1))
 (segment (start 138.639999 95.825001) (end 140.260001 95.825001) (width 0.25) (layer F.Cu) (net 1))
 (segment (start 138.4 95.585002) (end 138.639999 95.825001) (width 0.25) (layer F.Cu) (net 1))
 (segment (start 138.4 95) (end 138.4 95.585002) (width 0.25) (layer F.Cu) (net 1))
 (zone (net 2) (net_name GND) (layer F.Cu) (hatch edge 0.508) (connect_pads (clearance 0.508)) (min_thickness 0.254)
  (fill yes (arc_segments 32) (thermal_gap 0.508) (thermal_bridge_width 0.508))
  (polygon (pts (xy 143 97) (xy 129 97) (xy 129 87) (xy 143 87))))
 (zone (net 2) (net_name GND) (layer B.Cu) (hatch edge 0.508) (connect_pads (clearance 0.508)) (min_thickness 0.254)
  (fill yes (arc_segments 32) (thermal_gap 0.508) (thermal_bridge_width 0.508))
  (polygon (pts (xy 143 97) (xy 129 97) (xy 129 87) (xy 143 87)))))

